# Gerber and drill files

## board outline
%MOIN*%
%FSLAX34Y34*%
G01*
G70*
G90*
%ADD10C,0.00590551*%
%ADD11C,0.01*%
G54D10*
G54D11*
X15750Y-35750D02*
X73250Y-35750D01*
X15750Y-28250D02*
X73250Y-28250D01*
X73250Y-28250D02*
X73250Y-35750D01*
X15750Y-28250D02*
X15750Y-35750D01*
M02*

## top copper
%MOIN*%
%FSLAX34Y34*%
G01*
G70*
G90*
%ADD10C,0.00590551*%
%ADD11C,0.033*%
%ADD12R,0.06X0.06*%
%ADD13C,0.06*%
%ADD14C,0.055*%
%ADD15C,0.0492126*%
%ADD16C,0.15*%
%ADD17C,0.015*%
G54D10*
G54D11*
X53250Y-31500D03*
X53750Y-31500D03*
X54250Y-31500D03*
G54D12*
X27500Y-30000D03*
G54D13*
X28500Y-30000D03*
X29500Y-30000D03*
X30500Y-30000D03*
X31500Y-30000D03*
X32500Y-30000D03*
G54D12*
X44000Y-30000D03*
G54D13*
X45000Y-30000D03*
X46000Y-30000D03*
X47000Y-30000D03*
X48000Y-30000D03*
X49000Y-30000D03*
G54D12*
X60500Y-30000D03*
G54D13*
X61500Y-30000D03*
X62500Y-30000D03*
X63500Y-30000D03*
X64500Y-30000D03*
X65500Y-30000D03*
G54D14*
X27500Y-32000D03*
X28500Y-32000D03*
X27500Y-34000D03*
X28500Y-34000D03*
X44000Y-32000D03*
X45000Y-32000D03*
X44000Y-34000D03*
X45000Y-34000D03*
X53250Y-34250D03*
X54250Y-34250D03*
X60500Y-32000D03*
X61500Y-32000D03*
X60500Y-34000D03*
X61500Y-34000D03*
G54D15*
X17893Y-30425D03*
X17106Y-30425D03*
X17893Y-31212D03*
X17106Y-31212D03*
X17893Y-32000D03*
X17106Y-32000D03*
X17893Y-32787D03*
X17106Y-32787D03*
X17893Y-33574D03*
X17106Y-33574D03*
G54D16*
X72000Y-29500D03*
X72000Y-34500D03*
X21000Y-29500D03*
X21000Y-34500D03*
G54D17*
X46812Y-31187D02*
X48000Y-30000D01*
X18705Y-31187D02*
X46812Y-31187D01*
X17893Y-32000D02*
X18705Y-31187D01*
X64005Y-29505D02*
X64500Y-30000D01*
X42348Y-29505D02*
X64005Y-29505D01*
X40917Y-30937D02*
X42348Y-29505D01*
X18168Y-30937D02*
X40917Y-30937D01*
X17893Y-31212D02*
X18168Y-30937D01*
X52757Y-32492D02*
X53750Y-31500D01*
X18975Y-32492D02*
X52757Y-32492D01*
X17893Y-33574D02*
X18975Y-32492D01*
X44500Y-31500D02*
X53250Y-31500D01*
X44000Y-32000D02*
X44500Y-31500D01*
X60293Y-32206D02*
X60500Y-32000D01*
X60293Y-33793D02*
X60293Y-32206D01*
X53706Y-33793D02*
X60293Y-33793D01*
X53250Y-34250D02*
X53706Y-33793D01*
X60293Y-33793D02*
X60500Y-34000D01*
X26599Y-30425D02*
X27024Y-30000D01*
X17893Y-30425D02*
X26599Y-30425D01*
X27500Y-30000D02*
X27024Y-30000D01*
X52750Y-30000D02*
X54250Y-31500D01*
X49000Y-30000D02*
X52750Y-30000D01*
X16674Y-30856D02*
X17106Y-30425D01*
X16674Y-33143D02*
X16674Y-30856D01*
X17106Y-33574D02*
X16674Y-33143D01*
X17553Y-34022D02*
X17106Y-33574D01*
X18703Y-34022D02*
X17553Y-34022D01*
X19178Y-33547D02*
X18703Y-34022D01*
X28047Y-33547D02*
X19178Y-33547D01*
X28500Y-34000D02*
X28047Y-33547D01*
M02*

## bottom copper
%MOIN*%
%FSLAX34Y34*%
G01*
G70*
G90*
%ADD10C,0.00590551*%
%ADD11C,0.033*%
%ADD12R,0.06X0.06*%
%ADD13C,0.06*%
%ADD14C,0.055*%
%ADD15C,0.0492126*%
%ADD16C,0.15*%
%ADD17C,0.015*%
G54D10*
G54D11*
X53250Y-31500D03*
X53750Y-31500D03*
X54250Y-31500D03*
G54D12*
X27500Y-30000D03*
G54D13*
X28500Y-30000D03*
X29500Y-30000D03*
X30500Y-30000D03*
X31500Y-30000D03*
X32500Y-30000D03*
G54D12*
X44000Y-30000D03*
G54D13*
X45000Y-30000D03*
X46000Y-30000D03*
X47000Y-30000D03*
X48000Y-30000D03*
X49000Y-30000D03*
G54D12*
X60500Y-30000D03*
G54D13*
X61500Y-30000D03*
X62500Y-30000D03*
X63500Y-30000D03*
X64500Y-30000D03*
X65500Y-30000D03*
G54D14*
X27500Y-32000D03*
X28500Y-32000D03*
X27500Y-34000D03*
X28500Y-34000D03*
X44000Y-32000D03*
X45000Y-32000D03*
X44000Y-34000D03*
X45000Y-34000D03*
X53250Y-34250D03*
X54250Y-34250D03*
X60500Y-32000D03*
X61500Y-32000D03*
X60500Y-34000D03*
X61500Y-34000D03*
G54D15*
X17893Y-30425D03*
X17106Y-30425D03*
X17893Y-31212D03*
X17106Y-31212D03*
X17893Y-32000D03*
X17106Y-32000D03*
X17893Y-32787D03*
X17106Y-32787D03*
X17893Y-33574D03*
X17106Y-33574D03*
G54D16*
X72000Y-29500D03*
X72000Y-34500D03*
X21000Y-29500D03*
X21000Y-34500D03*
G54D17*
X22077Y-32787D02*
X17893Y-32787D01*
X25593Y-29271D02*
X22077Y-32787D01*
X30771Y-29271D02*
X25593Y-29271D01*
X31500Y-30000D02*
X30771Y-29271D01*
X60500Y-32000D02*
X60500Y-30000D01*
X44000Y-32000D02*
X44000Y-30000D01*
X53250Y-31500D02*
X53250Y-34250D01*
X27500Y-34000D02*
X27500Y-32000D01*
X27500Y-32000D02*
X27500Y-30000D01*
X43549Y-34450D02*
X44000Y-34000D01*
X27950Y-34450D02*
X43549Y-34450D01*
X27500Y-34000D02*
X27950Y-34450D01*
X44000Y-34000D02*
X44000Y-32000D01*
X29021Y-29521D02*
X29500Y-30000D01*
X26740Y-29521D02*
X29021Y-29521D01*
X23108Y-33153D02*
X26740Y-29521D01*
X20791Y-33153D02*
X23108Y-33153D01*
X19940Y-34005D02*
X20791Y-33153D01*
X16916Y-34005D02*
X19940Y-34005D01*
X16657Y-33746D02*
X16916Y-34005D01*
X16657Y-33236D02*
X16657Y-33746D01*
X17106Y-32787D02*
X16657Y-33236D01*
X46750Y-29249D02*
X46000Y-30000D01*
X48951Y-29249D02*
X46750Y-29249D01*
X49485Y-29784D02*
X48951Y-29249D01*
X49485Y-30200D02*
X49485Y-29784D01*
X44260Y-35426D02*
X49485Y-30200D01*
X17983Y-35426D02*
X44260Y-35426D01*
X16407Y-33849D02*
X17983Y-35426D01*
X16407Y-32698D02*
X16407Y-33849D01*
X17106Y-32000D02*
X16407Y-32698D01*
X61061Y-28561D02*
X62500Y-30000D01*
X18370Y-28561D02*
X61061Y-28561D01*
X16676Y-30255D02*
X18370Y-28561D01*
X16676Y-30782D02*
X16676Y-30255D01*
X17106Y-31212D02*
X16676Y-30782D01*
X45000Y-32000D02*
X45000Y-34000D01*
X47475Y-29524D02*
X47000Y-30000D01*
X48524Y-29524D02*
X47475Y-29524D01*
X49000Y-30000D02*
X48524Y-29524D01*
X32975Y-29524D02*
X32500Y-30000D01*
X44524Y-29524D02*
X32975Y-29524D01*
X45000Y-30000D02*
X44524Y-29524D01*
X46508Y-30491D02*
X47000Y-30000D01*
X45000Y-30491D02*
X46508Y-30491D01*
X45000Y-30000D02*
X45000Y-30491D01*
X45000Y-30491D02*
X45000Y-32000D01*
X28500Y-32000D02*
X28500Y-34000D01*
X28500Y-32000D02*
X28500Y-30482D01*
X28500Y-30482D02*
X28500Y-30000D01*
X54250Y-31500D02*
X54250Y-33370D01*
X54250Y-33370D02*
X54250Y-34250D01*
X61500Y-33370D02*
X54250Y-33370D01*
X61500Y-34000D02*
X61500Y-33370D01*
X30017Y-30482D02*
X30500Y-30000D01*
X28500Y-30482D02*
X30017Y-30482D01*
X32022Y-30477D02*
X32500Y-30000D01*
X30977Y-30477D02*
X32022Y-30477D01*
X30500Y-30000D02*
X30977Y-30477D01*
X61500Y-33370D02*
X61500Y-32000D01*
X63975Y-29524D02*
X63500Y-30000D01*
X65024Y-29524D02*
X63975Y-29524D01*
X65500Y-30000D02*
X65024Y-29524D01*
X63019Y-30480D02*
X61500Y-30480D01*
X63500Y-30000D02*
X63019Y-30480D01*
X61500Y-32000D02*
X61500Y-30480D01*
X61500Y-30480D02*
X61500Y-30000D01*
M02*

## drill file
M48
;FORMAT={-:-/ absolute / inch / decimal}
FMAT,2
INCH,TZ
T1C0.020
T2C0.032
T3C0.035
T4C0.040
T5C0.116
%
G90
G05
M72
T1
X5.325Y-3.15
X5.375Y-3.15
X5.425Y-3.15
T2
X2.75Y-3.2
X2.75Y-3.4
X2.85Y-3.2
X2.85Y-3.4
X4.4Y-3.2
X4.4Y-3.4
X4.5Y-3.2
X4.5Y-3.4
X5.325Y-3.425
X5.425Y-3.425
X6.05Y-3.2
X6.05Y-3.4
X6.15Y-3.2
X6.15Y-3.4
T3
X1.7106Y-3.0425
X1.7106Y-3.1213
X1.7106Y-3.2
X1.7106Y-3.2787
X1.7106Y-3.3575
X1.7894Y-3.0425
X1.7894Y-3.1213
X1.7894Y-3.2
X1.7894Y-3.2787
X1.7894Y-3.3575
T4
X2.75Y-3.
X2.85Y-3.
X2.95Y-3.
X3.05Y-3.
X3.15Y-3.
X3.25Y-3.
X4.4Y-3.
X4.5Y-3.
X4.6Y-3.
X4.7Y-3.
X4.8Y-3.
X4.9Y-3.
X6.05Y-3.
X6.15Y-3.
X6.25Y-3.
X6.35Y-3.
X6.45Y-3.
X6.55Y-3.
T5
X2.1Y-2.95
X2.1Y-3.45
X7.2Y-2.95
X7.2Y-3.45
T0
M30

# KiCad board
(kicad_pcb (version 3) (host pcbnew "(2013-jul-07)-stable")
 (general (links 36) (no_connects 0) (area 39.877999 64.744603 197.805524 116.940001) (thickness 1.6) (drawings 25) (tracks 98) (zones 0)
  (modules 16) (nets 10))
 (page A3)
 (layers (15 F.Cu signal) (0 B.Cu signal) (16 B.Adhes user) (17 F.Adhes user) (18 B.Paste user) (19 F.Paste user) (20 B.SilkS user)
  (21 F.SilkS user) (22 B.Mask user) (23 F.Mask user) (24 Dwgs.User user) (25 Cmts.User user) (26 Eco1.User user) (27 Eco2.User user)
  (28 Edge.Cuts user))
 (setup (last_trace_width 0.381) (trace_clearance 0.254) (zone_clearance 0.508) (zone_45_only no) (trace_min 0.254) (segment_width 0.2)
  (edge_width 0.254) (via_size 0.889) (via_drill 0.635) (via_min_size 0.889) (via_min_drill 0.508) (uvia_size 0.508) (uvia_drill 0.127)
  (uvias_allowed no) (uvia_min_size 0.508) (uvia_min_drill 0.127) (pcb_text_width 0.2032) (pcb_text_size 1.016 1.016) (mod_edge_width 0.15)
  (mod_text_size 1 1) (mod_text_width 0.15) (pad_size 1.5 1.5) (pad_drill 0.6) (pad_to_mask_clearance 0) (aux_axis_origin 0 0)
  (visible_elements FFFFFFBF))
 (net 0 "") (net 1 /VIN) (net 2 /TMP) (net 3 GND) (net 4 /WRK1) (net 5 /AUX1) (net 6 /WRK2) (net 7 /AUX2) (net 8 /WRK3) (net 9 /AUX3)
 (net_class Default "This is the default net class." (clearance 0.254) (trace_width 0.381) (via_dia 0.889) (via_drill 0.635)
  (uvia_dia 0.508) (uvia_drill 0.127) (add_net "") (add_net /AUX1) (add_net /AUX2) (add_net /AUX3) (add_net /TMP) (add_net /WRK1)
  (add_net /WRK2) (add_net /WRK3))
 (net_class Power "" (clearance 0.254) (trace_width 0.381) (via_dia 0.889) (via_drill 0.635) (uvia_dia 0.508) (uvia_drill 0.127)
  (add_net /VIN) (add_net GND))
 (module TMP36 (layer F.Cu) (at 136.525 80.01)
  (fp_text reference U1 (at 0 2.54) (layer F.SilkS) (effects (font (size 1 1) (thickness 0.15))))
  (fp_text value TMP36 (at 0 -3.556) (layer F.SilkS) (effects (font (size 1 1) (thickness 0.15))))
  (pad 1 thru_hole circle (at -1.27 0) (size 0.8382 0.8382) (drill 0.508) (layers *.Cu *.Mask F.SilkS) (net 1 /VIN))
  (pad 2 thru_hole circle (at 0 0) (size 0.8382 0.8382) (drill 0.508) (layers *.Cu *.Mask F.SilkS) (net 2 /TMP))
  (pad 3 thru_hole circle (at 1.27 0) (size 0.8382 0.8382) (drill 0.508) (layers *.Cu *.Mask F.SilkS) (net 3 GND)))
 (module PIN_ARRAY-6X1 (layer F.Cu) (at 76.2 76.2)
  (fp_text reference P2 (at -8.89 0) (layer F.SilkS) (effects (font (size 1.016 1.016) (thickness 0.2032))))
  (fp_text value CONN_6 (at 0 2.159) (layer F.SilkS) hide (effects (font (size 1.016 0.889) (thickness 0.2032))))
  (pad 1 thru_hole rect (at -6.35 0) (size 1.524 1.524) (drill 1.016) (layers *.Cu *.Mask F.SilkS) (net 1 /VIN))
  (pad 2 thru_hole circle (at -3.81 0) (size 1.524 1.524) (drill 1.016) (layers *.Cu *.Mask F.SilkS) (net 3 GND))
  (pad 3 thru_hole circle (at -1.27 0) (size 1.524 1.524) (drill 1.016) (layers *.Cu *.Mask F.SilkS) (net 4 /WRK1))
  (pad 4 thru_hole circle (at 1.27 0) (size 1.524 1.524) (drill 1.016) (layers *.Cu *.Mask F.SilkS) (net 3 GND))
  (pad 5 thru_hole circle (at 3.81 0) (size 1.524 1.524) (drill 1.016) (layers *.Cu *.Mask F.SilkS) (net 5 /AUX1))
  (pad 6 thru_hole circle (at 6.35 0) (size 1.524 1.524) (drill 1.016) (layers *.Cu *.Mask F.SilkS) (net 3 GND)))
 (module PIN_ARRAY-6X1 (layer F.Cu) (at 118.11 76.2)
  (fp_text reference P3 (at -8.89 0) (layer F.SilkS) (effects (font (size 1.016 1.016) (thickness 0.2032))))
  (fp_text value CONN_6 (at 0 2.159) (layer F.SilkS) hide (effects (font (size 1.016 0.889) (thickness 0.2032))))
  (pad 1 thru_hole rect (at -6.35 0) (size 1.524 1.524) (drill 1.016) (layers *.Cu *.Mask F.SilkS) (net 1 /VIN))
  (pad 2 thru_hole circle (at -3.81 0) (size 1.524 1.524) (drill 1.016) (layers *.Cu *.Mask F.SilkS) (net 3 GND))
  (pad 3 thru_hole circle (at -1.27 0) (size 1.524 1.524) (drill 1.016) (layers *.Cu *.Mask F.SilkS) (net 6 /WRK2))
  (pad 4 thru_hole circle (at 1.27 0) (size 1.524 1.524) (drill 1.016) (layers *.Cu *.Mask F.SilkS) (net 3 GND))
  (pad 5 thru_hole circle (at 3.81 0) (size 1.524 1.524) (drill 1.016) (layers *.Cu *.Mask F.SilkS) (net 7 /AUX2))
  (pad 6 thru_hole circle (at 6.35 0) (size 1.524 1.524) (drill 1.016) (layers *.Cu *.Mask F.SilkS) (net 3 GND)))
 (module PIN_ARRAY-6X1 (layer F.Cu) (at 160.02 76.2)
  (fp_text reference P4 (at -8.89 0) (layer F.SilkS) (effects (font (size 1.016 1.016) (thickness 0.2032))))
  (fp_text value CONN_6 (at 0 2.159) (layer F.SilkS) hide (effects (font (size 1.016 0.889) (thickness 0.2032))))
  (pad 1 thru_hole rect (at -6.35 0) (size 1.524 1.524) (drill 1.016) (layers *.Cu *.Mask F.SilkS) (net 1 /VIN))
  (pad 2 thru_hole circle (at -3.81 0) (size 1.524 1.524) (drill 1.016) (layers *.Cu *.Mask F.SilkS) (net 3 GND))
  (pad 3 thru_hole circle (at -1.27 0) (size 1.524 1.524) (drill 1.016) (layers *.Cu *.Mask F.SilkS) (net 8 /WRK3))
  (pad 4 thru_hole circle (at 1.27 0) (size 1.524 1.524) (drill 1.016) (layers *.Cu *.Mask F.SilkS) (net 3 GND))
  (pad 5 thru_hole circle (at 3.81 0) (size 1.524 1.524) (drill 1.016) (layers *.Cu *.Mask F.SilkS) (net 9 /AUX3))
  (pad 6 thru_hole circle (at 6.35 0) (size 1.524 1.524) (drill 1.016) (layers *.Cu *.Mask F.SilkS) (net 3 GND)))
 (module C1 (layer F.Cu) (at 71.12 81.28)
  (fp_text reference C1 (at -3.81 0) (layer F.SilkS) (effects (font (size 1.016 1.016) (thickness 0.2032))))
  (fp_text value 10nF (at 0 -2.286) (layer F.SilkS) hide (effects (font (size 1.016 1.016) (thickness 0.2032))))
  (pad 1 thru_hole circle (at -1.27 0) (size 1.397 1.397) (drill 0.8128) (layers *.Cu *.Mask F.SilkS) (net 1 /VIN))
  (pad 2 thru_hole circle (at 1.27 0) (size 1.397 1.397) (drill 0.8128) (layers *.Cu *.Mask F.SilkS) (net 3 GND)))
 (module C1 (layer F.Cu) (at 71.12 86.36)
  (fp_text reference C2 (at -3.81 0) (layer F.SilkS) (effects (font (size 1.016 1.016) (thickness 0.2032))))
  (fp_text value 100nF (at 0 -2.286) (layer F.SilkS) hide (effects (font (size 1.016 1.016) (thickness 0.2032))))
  (pad 1 thru_hole circle (at -1.27 0) (size 1.397 1.397) (drill 0.8128) (layers *.Cu *.Mask F.SilkS) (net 1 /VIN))
  (pad 2 thru_hole circle (at 1.27 0) (size 1.397 1.397) (drill 0.8128) (layers *.Cu *.Mask F.SilkS) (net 3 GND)))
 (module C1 (layer F.Cu) (at 113.03 81.28)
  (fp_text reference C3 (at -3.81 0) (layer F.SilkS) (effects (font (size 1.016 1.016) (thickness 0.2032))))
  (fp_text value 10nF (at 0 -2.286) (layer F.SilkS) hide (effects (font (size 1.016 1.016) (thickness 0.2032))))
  (pad 1 thru_hole circle (at -1.27 0) (size 1.397 1.397) (drill 0.8128) (layers *.Cu *.Mask F.SilkS) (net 1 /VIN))
  (pad 2 thru_hole circle (at 1.27 0) (size 1.397 1.397) (drill 0.8128) (layers *.Cu *.Mask F.SilkS) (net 3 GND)))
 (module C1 (layer F.Cu) (at 113.03 86.36)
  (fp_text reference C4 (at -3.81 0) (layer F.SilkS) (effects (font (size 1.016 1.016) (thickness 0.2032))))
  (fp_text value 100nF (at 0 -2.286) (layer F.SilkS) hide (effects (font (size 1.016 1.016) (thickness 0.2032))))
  (pad 1 thru_hole circle (at -1.27 0) (size 1.397 1.397) (drill 0.8128) (layers *.Cu *.Mask F.SilkS) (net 1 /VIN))
  (pad 2 thru_hole circle (at 1.27 0) (size 1.397 1.397) (drill 0.8128) (layers *.Cu *.Mask F.SilkS) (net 3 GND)))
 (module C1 (layer F.Cu) (at 136.525 86.995)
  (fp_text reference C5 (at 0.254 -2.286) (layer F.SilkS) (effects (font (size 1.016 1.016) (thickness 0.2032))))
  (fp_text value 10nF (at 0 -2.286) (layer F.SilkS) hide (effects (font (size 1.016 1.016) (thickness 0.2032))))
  (pad 1 thru_hole circle (at -1.27 0) (size 1.397 1.397) (drill 0.8128) (layers *.Cu *.Mask F.SilkS) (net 1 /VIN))
  (pad 2 thru_hole circle (at 1.27 0) (size 1.397 1.397) (drill 0.8128) (layers *.Cu *.Mask F.SilkS) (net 3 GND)))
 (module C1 (layer F.Cu) (at 154.94 81.28)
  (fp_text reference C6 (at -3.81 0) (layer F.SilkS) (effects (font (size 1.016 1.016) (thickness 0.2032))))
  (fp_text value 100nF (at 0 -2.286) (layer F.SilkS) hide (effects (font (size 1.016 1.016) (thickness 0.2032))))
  (pad 1 thru_hole circle (at -1.27 0) (size 1.397 1.397) (drill 0.8128) (layers *.Cu *.Mask F.SilkS) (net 1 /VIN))
  (pad 2 thru_hole circle (at 1.27 0) (size 1.397 1.397) (drill 0.8128) (layers *.Cu *.Mask F.SilkS) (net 3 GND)))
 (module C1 (layer F.Cu) (at 154.94 86.36)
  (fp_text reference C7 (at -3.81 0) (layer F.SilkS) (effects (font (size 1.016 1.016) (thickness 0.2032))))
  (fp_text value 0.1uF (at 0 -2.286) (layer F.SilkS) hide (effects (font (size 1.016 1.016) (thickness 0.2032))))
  (pad 1 thru_hole circle (at -1.27 0) (size 1.397 1.397) (drill 0.8128) (layers *.Cu *.Mask F.SilkS) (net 1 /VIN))
  (pad 2 thru_hole circle (at 1.27 0) (size 1.397 1.397) (drill 0.8128) (layers *.Cu *.Mask F.SilkS) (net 3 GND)))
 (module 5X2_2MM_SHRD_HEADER (layer B.Cu) (at 44.45 81.28 270)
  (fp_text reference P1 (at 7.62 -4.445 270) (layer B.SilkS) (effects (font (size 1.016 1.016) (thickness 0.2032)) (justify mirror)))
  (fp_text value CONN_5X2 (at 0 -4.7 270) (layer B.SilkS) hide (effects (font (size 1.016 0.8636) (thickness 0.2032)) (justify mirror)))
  (pad 1 thru_hole circle (at -4 -1 270) (size 1.25 1.25) (drill 0.9) (layers *.Cu *.Mask B.SilkS) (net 1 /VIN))
  (pad 2 thru_hole circle (at -4 1 270) (size 1.25 1.25) (drill 0.9) (layers *.Cu *.Mask B.SilkS) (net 3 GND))
  (pad 3 thru_hole circle (at -2 -1 270) (size 1.25 1.25) (drill 0.9) (layers *.Cu *.Mask B.SilkS) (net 9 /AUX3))
  (pad 4 thru_hole circle (at -2 1 270) (size 1.25 1.25) (drill 0.9) (layers *.Cu *.Mask B.SilkS) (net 8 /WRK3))
  (pad 5 thru_hole circle (at 0 -1 270) (size 1.25 1.25) (drill 0.9) (layers *.Cu *.Mask B.SilkS) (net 7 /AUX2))
  (pad 6 thru_hole circle (at 0 1 270) (size 1.25 1.25) (drill 0.9) (layers *.Cu *.Mask B.SilkS) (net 6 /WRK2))
  (pad 7 thru_hole circle (at 2 -1 270) (size 1.25 1.25) (drill 0.9) (layers *.Cu *.Mask B.SilkS) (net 5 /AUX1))
  (pad 8 thru_hole circle (at 2 1 270) (size 1.25 1.25) (drill 0.9) (layers *.Cu *.Mask B.SilkS) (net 4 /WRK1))
  (pad 9 thru_hole circle (at 4 -1 270) (size 1.25 1.25) (drill 0.9) (layers *.Cu *.Mask B.SilkS) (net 2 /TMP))
  (pad 10 thru_hole circle (at 4 1 270) (size 1.25 1.25) (drill 0.9) (layers *.Cu *.Mask B.SilkS) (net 3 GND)))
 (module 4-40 (layer F.Cu) (at 182.88 74.93)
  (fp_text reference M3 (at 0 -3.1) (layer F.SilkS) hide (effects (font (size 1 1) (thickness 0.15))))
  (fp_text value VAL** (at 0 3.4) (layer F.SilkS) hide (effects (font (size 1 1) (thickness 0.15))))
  (pad "" thru_hole circle (at 0 0) (size 3.81 3.81) (drill 2.9464) (layers *.Cu *.Mask F.SilkS)))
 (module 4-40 (layer F.Cu) (at 182.88 87.63)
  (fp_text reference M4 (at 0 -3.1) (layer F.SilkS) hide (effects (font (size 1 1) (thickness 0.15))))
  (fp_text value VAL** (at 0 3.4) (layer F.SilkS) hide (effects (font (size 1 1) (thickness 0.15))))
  (pad "" thru_hole circle (at 0 0) (size 3.81 3.81) (drill 2.9464) (layers *.Cu *.Mask F.SilkS)))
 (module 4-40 (layer F.Cu) (at 53.34 74.93)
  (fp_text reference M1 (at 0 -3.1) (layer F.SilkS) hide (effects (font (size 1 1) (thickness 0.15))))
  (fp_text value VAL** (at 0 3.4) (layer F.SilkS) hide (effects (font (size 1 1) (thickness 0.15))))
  (pad "" thru_hole circle (at 0 0) (size 3.81 3.81) (drill 2.9464) (layers *.Cu *.Mask F.SilkS)))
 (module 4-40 (layer F.Cu) (at 53.34 87.63)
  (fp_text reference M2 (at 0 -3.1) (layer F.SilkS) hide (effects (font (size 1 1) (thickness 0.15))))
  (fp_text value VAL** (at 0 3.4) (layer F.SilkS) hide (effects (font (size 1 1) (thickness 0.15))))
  (pad "" thru_hole circle (at 0 0) (size 3.81 3.81) (drill 2.9464) (layers *.Cu *.Mask F.SilkS)))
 (gr_line (start 40.005 90.805) (end 186.055 90.805) (angle 90) (layer Edge.Cuts) (width 0.254))
 (gr_line (start 40.005 71.755) (end 186.055 71.755) (angle 90) (layer Edge.Cuts) (width 0.254))
 (gr_line (start 186.055 71.755) (end 186.055 90.805) (angle 90) (layer Edge.Cuts) (width 0.254))
 (gr_line (start 40.005 71.755) (end 40.005 90.805) (angle 90) (layer Edge.Cuts) (width 0.254))
 (segment (start 56.0773 83.28) (end 45.45 83.28) (width 0.381) (layer B.Cu) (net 5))
 (segment (start 65.0081 74.3492) (end 56.0773 83.28) (width 0.381) (layer B.Cu) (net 5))
 (segment (start 78.1592 74.3492) (end 65.0081 74.3492) (width 0.381) (layer B.Cu) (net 5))
 (segment (start 80.01 76.2) (end 78.1592 74.3492) (width 0.381) (layer B.Cu) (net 5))
 (segment (start 118.9032 79.2168) (end 121.92 76.2) (width 0.381) (layer F.Cu) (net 7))
 (segment (start 47.5132 79.2168) (end 118.9032 79.2168) (width 0.381) (layer F.Cu) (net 7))
 (segment (start 45.45 81.28) (end 47.5132 79.2168) (width 0.381) (layer F.Cu) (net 7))
 (segment (start 162.575 74.945) (end 163.83 76.2) (width 0.381) (layer F.Cu) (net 9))
 (segment (start 107.566 74.945) (end 162.575 74.945) (width 0.381) (layer F.Cu) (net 9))
 (segment (start 103.9295 78.5815) (end 107.566 74.945) (width 0.381) (layer F.Cu) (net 9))
 (segment (start 46.1485 78.5815) (end 103.9295 78.5815) (width 0.381) (layer F.Cu) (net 9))
 (segment (start 45.45 79.28) (end 46.1485 78.5815) (width 0.381) (layer F.Cu) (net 9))
 (segment (start 134.0038 82.5312) (end 136.525 80.01) (width 0.381) (layer F.Cu) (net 2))
 (segment (start 48.1988 82.5312) (end 134.0038 82.5312) (width 0.381) (layer F.Cu) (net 2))
 (segment (start 45.45 85.28) (end 48.1988 82.5312) (width 0.381) (layer F.Cu) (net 2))
 (segment (start 153.67 81.28) (end 153.67 76.2) (width 0.381) (layer B.Cu) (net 1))
 (segment (start 111.76 81.28) (end 111.76 76.2) (width 0.381) (layer B.Cu) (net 1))
 (segment (start 113.03 80.01) (end 135.255 80.01) (width 0.381) (layer F.Cu) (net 1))
 (segment (start 111.76 81.28) (end 113.03 80.01) (width 0.381) (layer F.Cu) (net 1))
 (segment (start 135.255 80.01) (end 135.255 86.995) (width 0.381) (layer B.Cu) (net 1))
 (segment (start 153.1451 81.8049) (end 153.67 81.28) (width 0.381) (layer F.Cu) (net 1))
 (segment (start 153.1451 85.8351) (end 153.1451 81.8049) (width 0.381) (layer F.Cu) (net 1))
 (segment (start 136.4149 85.8351) (end 153.1451 85.8351) (width 0.381) (layer F.Cu) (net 1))
 (segment (start 135.255 86.995) (end 136.4149 85.8351) (width 0.381) (layer F.Cu) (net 1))
 (segment (start 153.1451 85.8351) (end 153.67 86.36) (width 0.381) (layer F.Cu) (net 1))
 (segment (start 69.85 86.36) (end 69.85 81.28) (width 0.381) (layer B.Cu) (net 1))
 (segment (start 69.85 81.28) (end 69.85 76.2) (width 0.381) (layer B.Cu) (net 1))
 (segment (start 67.5632 77.28) (end 68.6432 76.2) (width 0.381) (layer F.Cu) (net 1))
 (segment (start 45.45 77.28) (end 67.5632 77.28) (width 0.381) (layer F.Cu) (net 1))
 (segment (start 69.85 76.2) (end 68.6432 76.2) (width 0.381) (layer F.Cu) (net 1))
 (segment (start 110.6157 87.5043) (end 111.76 86.36) (width 0.381) (layer B.Cu) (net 1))
 (segment (start 70.9943 87.5043) (end 110.6157 87.5043) (width 0.381) (layer B.Cu) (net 1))
 (segment (start 69.85 86.36) (end 70.9943 87.5043) (width 0.381) (layer B.Cu) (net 1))
 (segment (start 111.76 86.36) (end 111.76 81.28) (width 0.381) (layer B.Cu) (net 1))
 (segment (start 73.7146 74.9846) (end 74.93 76.2) (width 0.381) (layer B.Cu) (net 4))
 (segment (start 67.9218 74.9846) (end 73.7146 74.9846) (width 0.381) (layer B.Cu) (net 4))
 (segment (start 58.6963 84.2101) (end 67.9218 74.9846) (width 0.381) (layer B.Cu) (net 4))
 (segment (start 52.8106 84.2101) (end 58.6963 84.2101) (width 0.381) (layer B.Cu) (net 4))
 (segment (start 50.6479 86.3728) (end 52.8106 84.2101) (width 0.381) (layer B.Cu) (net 4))
 (segment (start 42.9678 86.3728) (end 50.6479 86.3728) (width 0.381) (layer B.Cu) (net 4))
 (segment (start 42.3101 85.7151) (end 42.9678 86.3728) (width 0.381) (layer B.Cu) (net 4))
 (segment (start 42.3101 84.4199) (end 42.3101 85.7151) (width 0.381) (layer B.Cu) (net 4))
 (segment (start 43.45 83.28) (end 42.3101 84.4199) (width 0.381) (layer B.Cu) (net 4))
 (segment (start 118.7453 74.2947) (end 116.84 76.2) (width 0.381) (layer B.Cu) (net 6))
 (segment (start 124.3371 74.2947) (end 118.7453 74.2947) (width 0.381) (layer B.Cu) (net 6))
 (segment (start 125.6941 75.6517) (end 124.3371 74.2947) (width 0.381) (layer B.Cu) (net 6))
 (segment (start 125.6941 76.7103) (end 125.6941 75.6517) (width 0.381) (layer B.Cu) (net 6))
 (segment (start 112.4216 89.9828) (end 125.6941 76.7103) (width 0.381) (layer B.Cu) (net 6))
 (segment (start 45.6792 89.9828) (end 112.4216 89.9828) (width 0.381) (layer B.Cu) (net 6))
 (segment (start 41.6747 85.9783) (end 45.6792 89.9828) (width 0.381) (layer B.Cu) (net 6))
 (segment (start 41.6747 83.0553) (end 41.6747 85.9783) (width 0.381) (layer B.Cu) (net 6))
 (segment (start 43.45 81.28) (end 41.6747 83.0553) (width 0.381) (layer B.Cu) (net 6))
 (segment (start 155.096 72.546) (end 158.75 76.2) (width 0.381) (layer B.Cu) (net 8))
 (segment (start 46.6602 72.546) (end 155.096 72.546) (width 0.381) (layer B.Cu) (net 8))
 (segment (start 42.3571 76.8491) (end 46.6602 72.546) (width 0.381) (layer B.Cu) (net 8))
 (segment (start 42.3571 78.1871) (end 42.3571 76.8491) (width 0.381) (layer B.Cu) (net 8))
 (segment (start 43.45 79.28) (end 42.3571 78.1871) (width 0.381) (layer B.Cu) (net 8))
 (segment (start 114.3 81.28) (end 114.3 86.36) (width 0.381) (layer B.Cu) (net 3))
 (segment (start 120.5869 74.9931) (end 119.38 76.2) (width 0.381) (layer B.Cu) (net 3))
 (segment (start 123.2531 74.9931) (end 120.5869 74.9931) (width 0.381) (layer B.Cu) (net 3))
 (segment (start 124.46 76.2) (end 123.2531 74.9931) (width 0.381) (layer B.Cu) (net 3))
 (segment (start 83.7569 74.9931) (end 82.55 76.2) (width 0.381) (layer B.Cu) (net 3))
 (segment (start 113.0931 74.9931) (end 83.7569 74.9931) (width 0.381) (layer B.Cu) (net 3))
 (segment (start 114.3 76.2) (end 113.0931 74.9931) (width 0.381) (layer B.Cu) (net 3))
 (segment (start 118.1316 77.4484) (end 119.38 76.2) (width 0.381) (layer B.Cu) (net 3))
 (segment (start 114.3 77.4484) (end 118.1316 77.4484) (width 0.381) (layer B.Cu) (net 3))
 (segment (start 114.3 76.2) (end 114.3 77.4484) (width 0.381) (layer B.Cu) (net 3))
 (segment (start 114.3 77.4484) (end 114.3 81.28) (width 0.381) (layer B.Cu) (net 3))
 (segment (start 133.985 76.2) (end 137.795 80.01) (width 0.381) (layer F.Cu) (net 3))
 (segment (start 124.46 76.2) (end 133.985 76.2) (width 0.381) (layer F.Cu) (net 3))
 (segment (start 72.39 81.28) (end 72.39 86.36) (width 0.381) (layer B.Cu) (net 3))
 (segment (start 72.39 81.28) (end 72.39 77.4262) (width 0.381) (layer B.Cu) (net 3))
 (segment (start 72.39 77.4262) (end 72.39 76.2) (width 0.381) (layer B.Cu) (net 3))
 (segment (start 137.795 80.01) (end 137.795 84.7601) (width 0.381) (layer B.Cu) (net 3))
 (segment (start 137.795 84.7601) (end 137.795 86.995) (width 0.381) (layer B.Cu) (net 3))
 (segment (start 156.21 84.7601) (end 137.795 84.7601) (width 0.381) (layer B.Cu) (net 3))
 (segment (start 156.21 86.36) (end 156.21 84.7601) (width 0.381) (layer B.Cu) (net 3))
 (segment (start 42.3542 78.3758) (end 43.45 77.28) (width 0.381) (layer F.Cu) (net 3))
 (segment (start 42.3542 84.1842) (end 42.3542 78.3758) (width 0.381) (layer F.Cu) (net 3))
 (segment (start 43.45 85.28) (end 42.3542 84.1842) (width 0.381) (layer F.Cu) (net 3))
 (segment (start 44.5862 86.4162) (end 43.45 85.28) (width 0.381) (layer F.Cu) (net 3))
 (segment (start 47.5078 86.4162) (end 44.5862 86.4162) (width 0.381) (layer F.Cu) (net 3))
 (segment (start 48.7139 85.2101) (end 47.5078 86.4162) (width 0.381) (layer F.Cu) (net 3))
 (segment (start 71.2401 85.2101) (end 48.7139 85.2101) (width 0.381) (layer F.Cu) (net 3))
 (segment (start 72.39 86.36) (end 71.2401 85.2101) (width 0.381) (layer F.Cu) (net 3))
 (segment (start 76.2438 77.4262) (end 77.47 76.2) (width 0.381) (layer B.Cu) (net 3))
 (segment (start 72.39 77.4262) (end 76.2438 77.4262) (width 0.381) (layer B.Cu) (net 3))
 (segment (start 81.3371 77.4129) (end 82.55 76.2) (width 0.381) (layer B.Cu) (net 3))
 (segment (start 78.6829 77.4129) (end 81.3371 77.4129) (width 0.381) (layer B.Cu) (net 3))
 (segment (start 77.47 76.2) (end 78.6829 77.4129) (width 0.381) (layer B.Cu) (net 3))
 (segment (start 156.21 84.7601) (end 156.21 81.28) (width 0.381) (layer B.Cu) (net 3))
 (segment (start 162.4969 74.9931) (end 161.29 76.2) (width 0.381) (layer B.Cu) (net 3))
 (segment (start 165.1631 74.9931) (end 162.4969 74.9931) (width 0.381) (layer B.Cu) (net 3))
 (segment (start 166.37 76.2) (end 165.1631 74.9931) (width 0.381) (layer B.Cu) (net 3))
 (segment (start 160.0705 77.4195) (end 156.21 77.4195) (width 0.381) (layer B.Cu) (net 3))
 (segment (start 161.29 76.2) (end 160.0705 77.4195) (width 0.381) (layer B.Cu) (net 3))
 (segment (start 156.21 81.28) (end 156.21 77.4195) (width 0.381) (layer B.Cu) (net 3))
 (segment (start 156.21 77.4195) (end 156.21 76.2) (width 0.381) (layer B.Cu) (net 3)))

